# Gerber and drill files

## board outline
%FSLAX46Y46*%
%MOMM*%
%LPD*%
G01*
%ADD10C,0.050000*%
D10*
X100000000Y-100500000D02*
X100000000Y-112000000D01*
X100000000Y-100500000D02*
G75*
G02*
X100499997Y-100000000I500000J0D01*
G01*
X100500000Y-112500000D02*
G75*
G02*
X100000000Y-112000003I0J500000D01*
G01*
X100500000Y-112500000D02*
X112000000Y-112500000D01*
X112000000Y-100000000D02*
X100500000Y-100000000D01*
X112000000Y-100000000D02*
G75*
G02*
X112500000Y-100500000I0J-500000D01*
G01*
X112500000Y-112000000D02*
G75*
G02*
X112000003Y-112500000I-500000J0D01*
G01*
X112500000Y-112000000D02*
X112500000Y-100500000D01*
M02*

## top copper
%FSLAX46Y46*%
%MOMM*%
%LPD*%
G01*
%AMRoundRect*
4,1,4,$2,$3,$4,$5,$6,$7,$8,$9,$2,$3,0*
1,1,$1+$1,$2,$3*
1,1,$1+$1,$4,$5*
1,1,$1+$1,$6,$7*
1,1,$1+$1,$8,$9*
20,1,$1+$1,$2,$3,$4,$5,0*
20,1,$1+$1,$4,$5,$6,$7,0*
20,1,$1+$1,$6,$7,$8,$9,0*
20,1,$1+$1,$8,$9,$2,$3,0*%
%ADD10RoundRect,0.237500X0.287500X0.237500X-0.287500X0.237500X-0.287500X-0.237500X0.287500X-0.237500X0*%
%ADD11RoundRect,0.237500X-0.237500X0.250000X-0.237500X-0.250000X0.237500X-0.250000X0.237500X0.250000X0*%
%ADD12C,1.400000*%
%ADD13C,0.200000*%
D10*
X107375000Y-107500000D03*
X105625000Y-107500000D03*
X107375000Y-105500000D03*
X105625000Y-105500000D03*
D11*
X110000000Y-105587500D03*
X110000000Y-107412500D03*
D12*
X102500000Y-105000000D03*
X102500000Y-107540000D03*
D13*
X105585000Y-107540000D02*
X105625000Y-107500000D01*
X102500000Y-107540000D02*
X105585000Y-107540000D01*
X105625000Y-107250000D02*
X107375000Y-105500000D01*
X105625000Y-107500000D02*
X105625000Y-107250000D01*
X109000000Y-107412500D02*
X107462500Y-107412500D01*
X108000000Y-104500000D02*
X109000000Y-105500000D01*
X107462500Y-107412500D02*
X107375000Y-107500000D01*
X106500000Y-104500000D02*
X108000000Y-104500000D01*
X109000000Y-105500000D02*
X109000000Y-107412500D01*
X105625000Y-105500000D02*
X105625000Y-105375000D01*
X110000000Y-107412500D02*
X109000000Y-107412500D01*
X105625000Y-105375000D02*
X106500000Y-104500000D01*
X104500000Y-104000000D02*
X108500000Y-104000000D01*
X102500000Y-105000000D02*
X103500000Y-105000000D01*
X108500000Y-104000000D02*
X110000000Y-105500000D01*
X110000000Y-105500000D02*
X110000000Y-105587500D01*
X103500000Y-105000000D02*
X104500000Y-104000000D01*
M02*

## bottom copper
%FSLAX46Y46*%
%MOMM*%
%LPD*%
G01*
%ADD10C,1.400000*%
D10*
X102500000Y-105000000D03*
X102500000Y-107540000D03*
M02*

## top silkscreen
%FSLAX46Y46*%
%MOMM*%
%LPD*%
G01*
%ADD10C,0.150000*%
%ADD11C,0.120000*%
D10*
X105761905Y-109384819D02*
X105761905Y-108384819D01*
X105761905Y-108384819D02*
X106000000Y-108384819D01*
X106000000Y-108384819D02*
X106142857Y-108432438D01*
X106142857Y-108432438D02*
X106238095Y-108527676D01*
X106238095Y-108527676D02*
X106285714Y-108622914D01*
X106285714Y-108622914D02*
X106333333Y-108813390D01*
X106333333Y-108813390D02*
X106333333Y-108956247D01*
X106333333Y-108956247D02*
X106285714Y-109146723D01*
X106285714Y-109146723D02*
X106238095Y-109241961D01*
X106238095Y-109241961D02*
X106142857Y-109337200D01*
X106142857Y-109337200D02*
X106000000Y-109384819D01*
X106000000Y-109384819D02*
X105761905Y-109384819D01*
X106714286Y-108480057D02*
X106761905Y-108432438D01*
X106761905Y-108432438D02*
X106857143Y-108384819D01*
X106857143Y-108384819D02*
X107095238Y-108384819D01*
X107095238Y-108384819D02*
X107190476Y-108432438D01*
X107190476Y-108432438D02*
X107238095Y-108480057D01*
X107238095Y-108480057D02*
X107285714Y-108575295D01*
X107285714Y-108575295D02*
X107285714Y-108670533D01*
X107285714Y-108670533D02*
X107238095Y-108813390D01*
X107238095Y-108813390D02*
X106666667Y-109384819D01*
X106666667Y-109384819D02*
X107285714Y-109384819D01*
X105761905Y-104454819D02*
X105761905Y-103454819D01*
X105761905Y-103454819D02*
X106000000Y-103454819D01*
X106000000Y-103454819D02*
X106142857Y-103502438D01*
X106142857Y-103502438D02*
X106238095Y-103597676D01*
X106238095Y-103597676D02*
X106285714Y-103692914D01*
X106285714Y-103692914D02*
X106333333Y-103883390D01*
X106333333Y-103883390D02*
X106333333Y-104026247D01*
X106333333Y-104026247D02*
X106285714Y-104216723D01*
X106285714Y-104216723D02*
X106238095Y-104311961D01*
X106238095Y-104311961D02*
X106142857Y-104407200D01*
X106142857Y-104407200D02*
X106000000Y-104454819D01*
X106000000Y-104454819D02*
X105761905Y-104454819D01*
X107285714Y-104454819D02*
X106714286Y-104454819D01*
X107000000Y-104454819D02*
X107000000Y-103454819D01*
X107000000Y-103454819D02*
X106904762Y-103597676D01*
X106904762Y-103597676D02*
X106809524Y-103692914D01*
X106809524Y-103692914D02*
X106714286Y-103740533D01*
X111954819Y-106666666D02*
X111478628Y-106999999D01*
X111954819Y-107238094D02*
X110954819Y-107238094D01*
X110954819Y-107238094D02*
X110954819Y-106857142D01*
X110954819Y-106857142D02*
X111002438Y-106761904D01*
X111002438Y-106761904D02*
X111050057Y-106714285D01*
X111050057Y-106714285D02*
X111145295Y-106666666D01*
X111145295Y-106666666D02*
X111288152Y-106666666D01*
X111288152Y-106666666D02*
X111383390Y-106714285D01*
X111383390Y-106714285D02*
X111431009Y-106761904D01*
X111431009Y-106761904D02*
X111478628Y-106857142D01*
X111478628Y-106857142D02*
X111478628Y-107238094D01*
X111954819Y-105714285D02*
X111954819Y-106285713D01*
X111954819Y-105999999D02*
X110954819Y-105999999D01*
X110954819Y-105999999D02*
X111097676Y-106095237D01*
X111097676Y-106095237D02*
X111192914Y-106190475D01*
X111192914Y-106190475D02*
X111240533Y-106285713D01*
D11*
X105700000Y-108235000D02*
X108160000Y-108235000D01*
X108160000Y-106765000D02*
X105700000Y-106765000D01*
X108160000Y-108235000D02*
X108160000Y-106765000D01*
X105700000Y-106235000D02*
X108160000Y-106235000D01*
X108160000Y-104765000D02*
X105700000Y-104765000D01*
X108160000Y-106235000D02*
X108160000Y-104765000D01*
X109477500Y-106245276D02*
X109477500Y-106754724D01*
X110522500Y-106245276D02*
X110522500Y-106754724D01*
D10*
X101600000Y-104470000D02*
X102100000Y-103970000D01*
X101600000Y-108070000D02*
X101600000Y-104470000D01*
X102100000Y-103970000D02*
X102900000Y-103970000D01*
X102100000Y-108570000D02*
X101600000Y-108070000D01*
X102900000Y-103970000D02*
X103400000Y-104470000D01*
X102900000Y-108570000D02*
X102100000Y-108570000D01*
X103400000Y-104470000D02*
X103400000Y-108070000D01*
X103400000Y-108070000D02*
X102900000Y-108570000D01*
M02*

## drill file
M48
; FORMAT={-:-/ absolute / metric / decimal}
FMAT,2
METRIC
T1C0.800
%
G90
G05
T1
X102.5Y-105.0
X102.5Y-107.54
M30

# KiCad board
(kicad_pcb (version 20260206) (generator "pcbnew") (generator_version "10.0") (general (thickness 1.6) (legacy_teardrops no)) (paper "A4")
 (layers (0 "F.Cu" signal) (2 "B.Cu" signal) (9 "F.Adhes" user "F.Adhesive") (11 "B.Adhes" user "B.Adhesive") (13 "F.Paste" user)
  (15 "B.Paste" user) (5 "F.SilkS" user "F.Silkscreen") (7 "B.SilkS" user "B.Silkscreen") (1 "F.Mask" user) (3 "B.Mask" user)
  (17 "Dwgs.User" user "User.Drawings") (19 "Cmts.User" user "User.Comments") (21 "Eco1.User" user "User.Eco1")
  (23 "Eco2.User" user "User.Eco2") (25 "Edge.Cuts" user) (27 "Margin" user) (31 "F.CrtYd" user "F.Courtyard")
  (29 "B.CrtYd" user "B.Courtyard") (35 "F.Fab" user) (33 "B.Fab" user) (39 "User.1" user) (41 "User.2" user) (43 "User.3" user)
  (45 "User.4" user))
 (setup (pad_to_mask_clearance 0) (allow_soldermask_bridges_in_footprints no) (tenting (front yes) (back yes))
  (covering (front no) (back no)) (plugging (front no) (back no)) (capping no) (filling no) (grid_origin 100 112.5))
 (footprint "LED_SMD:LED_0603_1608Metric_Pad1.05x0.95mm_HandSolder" (layer "F.Cu") (at 106.5 107.5 180)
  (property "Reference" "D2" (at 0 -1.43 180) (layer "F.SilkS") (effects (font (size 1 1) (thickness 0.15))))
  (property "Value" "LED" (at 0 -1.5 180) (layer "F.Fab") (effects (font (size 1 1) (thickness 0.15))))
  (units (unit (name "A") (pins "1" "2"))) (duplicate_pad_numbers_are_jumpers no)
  (fp_line (start 0.8 -0.735) (end -1.66 -0.735) (stroke (width 0.12) (type solid)) (layer "F.SilkS"))
  (fp_line (start -1.66 0.735) (end 0.8 0.735) (stroke (width 0.12) (type solid)) (layer "F.SilkS"))
  (fp_line (start -1.66 -0.735) (end -1.66 0.735) (stroke (width 0.12) (type solid)) (layer "F.SilkS"))
  (pad "1" smd roundrect (at -0.875 0 180) (size 1.05 0.95) (layers "F.Cu" "F.Mask" "F.Paste") (roundrect_rratio 0.25) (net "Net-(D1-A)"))
  (pad "2" smd roundrect (at 0.875 0 180) (size 1.05 0.95) (layers "F.Cu" "F.Mask" "F.Paste") (roundrect_rratio 0.25) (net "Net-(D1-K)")))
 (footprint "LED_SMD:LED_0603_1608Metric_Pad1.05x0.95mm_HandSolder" (layer "F.Cu") (at 106.5 105.5 180)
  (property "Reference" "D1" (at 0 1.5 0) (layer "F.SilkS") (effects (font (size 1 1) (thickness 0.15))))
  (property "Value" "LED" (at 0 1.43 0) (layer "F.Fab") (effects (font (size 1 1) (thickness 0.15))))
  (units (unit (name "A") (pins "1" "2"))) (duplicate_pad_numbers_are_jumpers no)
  (fp_line (start 0.8 -0.735) (end -1.66 -0.735) (stroke (width 0.12) (type solid)) (layer "F.SilkS"))
  (fp_line (start -1.66 0.735) (end 0.8 0.735) (stroke (width 0.12) (type solid)) (layer "F.SilkS"))
  (fp_line (start -1.66 -0.735) (end -1.66 0.735) (stroke (width 0.12) (type solid)) (layer "F.SilkS"))
  (pad "1" smd roundrect (at -0.875 0 180) (size 1.05 0.95) (layers "F.Cu" "F.Mask" "F.Paste") (roundrect_rratio 0.25) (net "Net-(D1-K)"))
  (pad "2" smd roundrect (at 0.875 0 180) (size 1.05 0.95) (layers "F.Cu" "F.Mask" "F.Paste") (roundrect_rratio 0.25) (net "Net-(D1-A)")))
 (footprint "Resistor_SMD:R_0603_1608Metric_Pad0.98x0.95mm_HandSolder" (layer "F.Cu") (at 110 106.5 -90)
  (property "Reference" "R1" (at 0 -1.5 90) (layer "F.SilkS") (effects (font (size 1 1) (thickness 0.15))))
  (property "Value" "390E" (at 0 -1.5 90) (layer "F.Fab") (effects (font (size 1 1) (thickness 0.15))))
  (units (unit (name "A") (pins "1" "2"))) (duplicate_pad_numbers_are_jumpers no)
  (fp_line (start -0.254724 0.5225) (end 0.254724 0.5225) (stroke (width 0.12) (type solid)) (layer "F.SilkS"))
  (fp_line (start -0.254724 -0.5225) (end 0.254724 -0.5225) (stroke (width 0.12) (type solid)) (layer "F.SilkS"))
  (pad "1" smd roundrect (at -0.9125 0 270) (size 0.975 0.95) (layers "F.Cu" "F.Mask" "F.Paste") (roundrect_rratio 0.25)
   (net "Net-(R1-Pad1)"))
  (pad "2" smd roundrect (at 0.9125 0 270) (size 0.975 0.95) (layers "F.Cu" "F.Mask" "F.Paste") (roundrect_rratio 0.25) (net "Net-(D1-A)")))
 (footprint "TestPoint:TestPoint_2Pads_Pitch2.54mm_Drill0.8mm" (layer "F.Cu") (at 102.5 105 -90)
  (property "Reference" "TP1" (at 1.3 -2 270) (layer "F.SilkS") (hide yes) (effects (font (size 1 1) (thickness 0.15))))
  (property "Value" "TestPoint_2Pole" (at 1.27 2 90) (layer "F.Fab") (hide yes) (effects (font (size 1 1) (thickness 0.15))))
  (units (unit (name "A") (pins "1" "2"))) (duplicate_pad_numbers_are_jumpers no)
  (fp_line (start -0.53 0.9) (end -1.03 0.4) (stroke (width 0.15) (type solid)) (layer "F.SilkS"))
  (fp_line (start 3.07 0.9) (end -0.53 0.9) (stroke (width 0.15) (type solid)) (layer "F.SilkS"))
  (fp_line (start -1.03 0.4) (end -1.03 -0.4) (stroke (width 0.15) (type solid)) (layer "F.SilkS"))
  (fp_line (start 3.57 0.4) (end 3.07 0.9) (stroke (width 0.15) (type solid)) (layer "F.SilkS"))
  (fp_line (start -1.03 -0.4) (end -0.53 -0.9) (stroke (width 0.15) (type solid)) (layer "F.SilkS"))
  (fp_line (start 3.57 -0.4) (end 3.57 0.4) (stroke (width 0.15) (type solid)) (layer "F.SilkS"))
  (fp_line (start -0.53 -0.9) (end 3.07 -0.9) (stroke (width 0.15) (type solid)) (layer "F.SilkS"))
  (fp_line (start 3.07 -0.9) (end 3.57 -0.4) (stroke (width 0.15) (type solid)) (layer "F.SilkS"))
  (pad "1" thru_hole circle (at 0 0 270) (size 1.4 1.4) (drill 0.8) (layers "*.Cu" "*.Mask") (remove_unused_layers no) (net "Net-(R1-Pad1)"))
  (pad "2" thru_hole circle (at 2.54 0 270) (size 1.4 1.4) (drill 0.8) (layers "*.Cu" "*.Mask") (remove_unused_layers no) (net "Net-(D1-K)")))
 (gr_line (start 100 100.5) (end 100 112) (stroke (width 0.05) (type solid)) (layer "Edge.Cuts"))
 (gr_arc (start 100 100.5) (mid 100.146446 100.146448) (end 100.499997 100) (stroke (width 0.05) (type solid)) (layer "Edge.Cuts"))
 (gr_arc (start 100.5 112.5) (mid 100.146448 112.353554) (end 100 112.000003) (stroke (width 0.05) (type solid)) (layer "Edge.Cuts"))
 (gr_line (start 100.5 112.5) (end 112 112.5) (stroke (width 0.05) (type solid)) (layer "Edge.Cuts"))
 (gr_line (start 112 100) (end 100.5 100) (stroke (width 0.05) (type solid)) (layer "Edge.Cuts"))
 (gr_arc (start 112 100) (mid 112.353553 100.146447) (end 112.5 100.5) (stroke (width 0.05) (type solid)) (layer "Edge.Cuts"))
 (gr_arc (start 112.5 112) (mid 112.353554 112.353552) (end 112.000003 112.5) (stroke (width 0.05) (type solid)) (layer "Edge.Cuts"))
 (gr_line (start 112.5 112) (end 112.5 100.5) (stroke (width 0.05) (type default)) (layer "Edge.Cuts"))
 (segment (start 105.585 107.54) (end 105.625 107.5) (width 0.2) (layer "F.Cu") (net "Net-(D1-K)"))
 (segment (start 102.5 107.54) (end 105.585 107.54) (width 0.2) (layer "F.Cu") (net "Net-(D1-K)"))
 (segment (start 105.625 107.25) (end 107.375 105.5) (width 0.2) (layer "F.Cu") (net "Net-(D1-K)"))
 (segment (start 105.625 107.5) (end 105.625 107.25) (width 0.2) (layer "F.Cu") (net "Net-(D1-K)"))
 (segment (start 109 107.4125) (end 107.4625 107.4125) (width 0.2) (layer "F.Cu") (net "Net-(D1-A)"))
 (segment (start 108 104.5) (end 109 105.5) (width 0.2) (layer "F.Cu") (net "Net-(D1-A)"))
 (segment (start 107.4625 107.4125) (end 107.375 107.5) (width 0.2) (layer "F.Cu") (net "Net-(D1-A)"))
 (segment (start 106.5 104.5) (end 108 104.5) (width 0.2) (layer "F.Cu") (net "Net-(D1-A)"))
 (segment (start 109 105.5) (end 109 107.4125) (width 0.2) (layer "F.Cu") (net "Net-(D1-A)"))
 (segment (start 105.625 105.5) (end 105.625 105.375) (width 0.2) (layer "F.Cu") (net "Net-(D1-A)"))
 (segment (start 110 107.4125) (end 109 107.4125) (width 0.2) (layer "F.Cu") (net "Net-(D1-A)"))
 (segment (start 105.625 105.375) (end 106.5 104.5) (width 0.2) (layer "F.Cu") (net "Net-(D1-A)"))
 (segment (start 104.5 104) (end 108.5 104) (width 0.2) (layer "F.Cu") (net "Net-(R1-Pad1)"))
 (segment (start 102.5 105) (end 103.5 105) (width 0.2) (layer "F.Cu") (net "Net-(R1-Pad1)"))
 (segment (start 108.5 104) (end 110 105.5) (width 0.2) (layer "F.Cu") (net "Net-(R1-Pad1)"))
 (segment (start 110 105.5) (end 110 105.5875) (width 0.2) (layer "F.Cu") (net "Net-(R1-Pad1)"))
 (segment (start 103.5 105) (end 104.5 104) (width 0.2) (layer "F.Cu") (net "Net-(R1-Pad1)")))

